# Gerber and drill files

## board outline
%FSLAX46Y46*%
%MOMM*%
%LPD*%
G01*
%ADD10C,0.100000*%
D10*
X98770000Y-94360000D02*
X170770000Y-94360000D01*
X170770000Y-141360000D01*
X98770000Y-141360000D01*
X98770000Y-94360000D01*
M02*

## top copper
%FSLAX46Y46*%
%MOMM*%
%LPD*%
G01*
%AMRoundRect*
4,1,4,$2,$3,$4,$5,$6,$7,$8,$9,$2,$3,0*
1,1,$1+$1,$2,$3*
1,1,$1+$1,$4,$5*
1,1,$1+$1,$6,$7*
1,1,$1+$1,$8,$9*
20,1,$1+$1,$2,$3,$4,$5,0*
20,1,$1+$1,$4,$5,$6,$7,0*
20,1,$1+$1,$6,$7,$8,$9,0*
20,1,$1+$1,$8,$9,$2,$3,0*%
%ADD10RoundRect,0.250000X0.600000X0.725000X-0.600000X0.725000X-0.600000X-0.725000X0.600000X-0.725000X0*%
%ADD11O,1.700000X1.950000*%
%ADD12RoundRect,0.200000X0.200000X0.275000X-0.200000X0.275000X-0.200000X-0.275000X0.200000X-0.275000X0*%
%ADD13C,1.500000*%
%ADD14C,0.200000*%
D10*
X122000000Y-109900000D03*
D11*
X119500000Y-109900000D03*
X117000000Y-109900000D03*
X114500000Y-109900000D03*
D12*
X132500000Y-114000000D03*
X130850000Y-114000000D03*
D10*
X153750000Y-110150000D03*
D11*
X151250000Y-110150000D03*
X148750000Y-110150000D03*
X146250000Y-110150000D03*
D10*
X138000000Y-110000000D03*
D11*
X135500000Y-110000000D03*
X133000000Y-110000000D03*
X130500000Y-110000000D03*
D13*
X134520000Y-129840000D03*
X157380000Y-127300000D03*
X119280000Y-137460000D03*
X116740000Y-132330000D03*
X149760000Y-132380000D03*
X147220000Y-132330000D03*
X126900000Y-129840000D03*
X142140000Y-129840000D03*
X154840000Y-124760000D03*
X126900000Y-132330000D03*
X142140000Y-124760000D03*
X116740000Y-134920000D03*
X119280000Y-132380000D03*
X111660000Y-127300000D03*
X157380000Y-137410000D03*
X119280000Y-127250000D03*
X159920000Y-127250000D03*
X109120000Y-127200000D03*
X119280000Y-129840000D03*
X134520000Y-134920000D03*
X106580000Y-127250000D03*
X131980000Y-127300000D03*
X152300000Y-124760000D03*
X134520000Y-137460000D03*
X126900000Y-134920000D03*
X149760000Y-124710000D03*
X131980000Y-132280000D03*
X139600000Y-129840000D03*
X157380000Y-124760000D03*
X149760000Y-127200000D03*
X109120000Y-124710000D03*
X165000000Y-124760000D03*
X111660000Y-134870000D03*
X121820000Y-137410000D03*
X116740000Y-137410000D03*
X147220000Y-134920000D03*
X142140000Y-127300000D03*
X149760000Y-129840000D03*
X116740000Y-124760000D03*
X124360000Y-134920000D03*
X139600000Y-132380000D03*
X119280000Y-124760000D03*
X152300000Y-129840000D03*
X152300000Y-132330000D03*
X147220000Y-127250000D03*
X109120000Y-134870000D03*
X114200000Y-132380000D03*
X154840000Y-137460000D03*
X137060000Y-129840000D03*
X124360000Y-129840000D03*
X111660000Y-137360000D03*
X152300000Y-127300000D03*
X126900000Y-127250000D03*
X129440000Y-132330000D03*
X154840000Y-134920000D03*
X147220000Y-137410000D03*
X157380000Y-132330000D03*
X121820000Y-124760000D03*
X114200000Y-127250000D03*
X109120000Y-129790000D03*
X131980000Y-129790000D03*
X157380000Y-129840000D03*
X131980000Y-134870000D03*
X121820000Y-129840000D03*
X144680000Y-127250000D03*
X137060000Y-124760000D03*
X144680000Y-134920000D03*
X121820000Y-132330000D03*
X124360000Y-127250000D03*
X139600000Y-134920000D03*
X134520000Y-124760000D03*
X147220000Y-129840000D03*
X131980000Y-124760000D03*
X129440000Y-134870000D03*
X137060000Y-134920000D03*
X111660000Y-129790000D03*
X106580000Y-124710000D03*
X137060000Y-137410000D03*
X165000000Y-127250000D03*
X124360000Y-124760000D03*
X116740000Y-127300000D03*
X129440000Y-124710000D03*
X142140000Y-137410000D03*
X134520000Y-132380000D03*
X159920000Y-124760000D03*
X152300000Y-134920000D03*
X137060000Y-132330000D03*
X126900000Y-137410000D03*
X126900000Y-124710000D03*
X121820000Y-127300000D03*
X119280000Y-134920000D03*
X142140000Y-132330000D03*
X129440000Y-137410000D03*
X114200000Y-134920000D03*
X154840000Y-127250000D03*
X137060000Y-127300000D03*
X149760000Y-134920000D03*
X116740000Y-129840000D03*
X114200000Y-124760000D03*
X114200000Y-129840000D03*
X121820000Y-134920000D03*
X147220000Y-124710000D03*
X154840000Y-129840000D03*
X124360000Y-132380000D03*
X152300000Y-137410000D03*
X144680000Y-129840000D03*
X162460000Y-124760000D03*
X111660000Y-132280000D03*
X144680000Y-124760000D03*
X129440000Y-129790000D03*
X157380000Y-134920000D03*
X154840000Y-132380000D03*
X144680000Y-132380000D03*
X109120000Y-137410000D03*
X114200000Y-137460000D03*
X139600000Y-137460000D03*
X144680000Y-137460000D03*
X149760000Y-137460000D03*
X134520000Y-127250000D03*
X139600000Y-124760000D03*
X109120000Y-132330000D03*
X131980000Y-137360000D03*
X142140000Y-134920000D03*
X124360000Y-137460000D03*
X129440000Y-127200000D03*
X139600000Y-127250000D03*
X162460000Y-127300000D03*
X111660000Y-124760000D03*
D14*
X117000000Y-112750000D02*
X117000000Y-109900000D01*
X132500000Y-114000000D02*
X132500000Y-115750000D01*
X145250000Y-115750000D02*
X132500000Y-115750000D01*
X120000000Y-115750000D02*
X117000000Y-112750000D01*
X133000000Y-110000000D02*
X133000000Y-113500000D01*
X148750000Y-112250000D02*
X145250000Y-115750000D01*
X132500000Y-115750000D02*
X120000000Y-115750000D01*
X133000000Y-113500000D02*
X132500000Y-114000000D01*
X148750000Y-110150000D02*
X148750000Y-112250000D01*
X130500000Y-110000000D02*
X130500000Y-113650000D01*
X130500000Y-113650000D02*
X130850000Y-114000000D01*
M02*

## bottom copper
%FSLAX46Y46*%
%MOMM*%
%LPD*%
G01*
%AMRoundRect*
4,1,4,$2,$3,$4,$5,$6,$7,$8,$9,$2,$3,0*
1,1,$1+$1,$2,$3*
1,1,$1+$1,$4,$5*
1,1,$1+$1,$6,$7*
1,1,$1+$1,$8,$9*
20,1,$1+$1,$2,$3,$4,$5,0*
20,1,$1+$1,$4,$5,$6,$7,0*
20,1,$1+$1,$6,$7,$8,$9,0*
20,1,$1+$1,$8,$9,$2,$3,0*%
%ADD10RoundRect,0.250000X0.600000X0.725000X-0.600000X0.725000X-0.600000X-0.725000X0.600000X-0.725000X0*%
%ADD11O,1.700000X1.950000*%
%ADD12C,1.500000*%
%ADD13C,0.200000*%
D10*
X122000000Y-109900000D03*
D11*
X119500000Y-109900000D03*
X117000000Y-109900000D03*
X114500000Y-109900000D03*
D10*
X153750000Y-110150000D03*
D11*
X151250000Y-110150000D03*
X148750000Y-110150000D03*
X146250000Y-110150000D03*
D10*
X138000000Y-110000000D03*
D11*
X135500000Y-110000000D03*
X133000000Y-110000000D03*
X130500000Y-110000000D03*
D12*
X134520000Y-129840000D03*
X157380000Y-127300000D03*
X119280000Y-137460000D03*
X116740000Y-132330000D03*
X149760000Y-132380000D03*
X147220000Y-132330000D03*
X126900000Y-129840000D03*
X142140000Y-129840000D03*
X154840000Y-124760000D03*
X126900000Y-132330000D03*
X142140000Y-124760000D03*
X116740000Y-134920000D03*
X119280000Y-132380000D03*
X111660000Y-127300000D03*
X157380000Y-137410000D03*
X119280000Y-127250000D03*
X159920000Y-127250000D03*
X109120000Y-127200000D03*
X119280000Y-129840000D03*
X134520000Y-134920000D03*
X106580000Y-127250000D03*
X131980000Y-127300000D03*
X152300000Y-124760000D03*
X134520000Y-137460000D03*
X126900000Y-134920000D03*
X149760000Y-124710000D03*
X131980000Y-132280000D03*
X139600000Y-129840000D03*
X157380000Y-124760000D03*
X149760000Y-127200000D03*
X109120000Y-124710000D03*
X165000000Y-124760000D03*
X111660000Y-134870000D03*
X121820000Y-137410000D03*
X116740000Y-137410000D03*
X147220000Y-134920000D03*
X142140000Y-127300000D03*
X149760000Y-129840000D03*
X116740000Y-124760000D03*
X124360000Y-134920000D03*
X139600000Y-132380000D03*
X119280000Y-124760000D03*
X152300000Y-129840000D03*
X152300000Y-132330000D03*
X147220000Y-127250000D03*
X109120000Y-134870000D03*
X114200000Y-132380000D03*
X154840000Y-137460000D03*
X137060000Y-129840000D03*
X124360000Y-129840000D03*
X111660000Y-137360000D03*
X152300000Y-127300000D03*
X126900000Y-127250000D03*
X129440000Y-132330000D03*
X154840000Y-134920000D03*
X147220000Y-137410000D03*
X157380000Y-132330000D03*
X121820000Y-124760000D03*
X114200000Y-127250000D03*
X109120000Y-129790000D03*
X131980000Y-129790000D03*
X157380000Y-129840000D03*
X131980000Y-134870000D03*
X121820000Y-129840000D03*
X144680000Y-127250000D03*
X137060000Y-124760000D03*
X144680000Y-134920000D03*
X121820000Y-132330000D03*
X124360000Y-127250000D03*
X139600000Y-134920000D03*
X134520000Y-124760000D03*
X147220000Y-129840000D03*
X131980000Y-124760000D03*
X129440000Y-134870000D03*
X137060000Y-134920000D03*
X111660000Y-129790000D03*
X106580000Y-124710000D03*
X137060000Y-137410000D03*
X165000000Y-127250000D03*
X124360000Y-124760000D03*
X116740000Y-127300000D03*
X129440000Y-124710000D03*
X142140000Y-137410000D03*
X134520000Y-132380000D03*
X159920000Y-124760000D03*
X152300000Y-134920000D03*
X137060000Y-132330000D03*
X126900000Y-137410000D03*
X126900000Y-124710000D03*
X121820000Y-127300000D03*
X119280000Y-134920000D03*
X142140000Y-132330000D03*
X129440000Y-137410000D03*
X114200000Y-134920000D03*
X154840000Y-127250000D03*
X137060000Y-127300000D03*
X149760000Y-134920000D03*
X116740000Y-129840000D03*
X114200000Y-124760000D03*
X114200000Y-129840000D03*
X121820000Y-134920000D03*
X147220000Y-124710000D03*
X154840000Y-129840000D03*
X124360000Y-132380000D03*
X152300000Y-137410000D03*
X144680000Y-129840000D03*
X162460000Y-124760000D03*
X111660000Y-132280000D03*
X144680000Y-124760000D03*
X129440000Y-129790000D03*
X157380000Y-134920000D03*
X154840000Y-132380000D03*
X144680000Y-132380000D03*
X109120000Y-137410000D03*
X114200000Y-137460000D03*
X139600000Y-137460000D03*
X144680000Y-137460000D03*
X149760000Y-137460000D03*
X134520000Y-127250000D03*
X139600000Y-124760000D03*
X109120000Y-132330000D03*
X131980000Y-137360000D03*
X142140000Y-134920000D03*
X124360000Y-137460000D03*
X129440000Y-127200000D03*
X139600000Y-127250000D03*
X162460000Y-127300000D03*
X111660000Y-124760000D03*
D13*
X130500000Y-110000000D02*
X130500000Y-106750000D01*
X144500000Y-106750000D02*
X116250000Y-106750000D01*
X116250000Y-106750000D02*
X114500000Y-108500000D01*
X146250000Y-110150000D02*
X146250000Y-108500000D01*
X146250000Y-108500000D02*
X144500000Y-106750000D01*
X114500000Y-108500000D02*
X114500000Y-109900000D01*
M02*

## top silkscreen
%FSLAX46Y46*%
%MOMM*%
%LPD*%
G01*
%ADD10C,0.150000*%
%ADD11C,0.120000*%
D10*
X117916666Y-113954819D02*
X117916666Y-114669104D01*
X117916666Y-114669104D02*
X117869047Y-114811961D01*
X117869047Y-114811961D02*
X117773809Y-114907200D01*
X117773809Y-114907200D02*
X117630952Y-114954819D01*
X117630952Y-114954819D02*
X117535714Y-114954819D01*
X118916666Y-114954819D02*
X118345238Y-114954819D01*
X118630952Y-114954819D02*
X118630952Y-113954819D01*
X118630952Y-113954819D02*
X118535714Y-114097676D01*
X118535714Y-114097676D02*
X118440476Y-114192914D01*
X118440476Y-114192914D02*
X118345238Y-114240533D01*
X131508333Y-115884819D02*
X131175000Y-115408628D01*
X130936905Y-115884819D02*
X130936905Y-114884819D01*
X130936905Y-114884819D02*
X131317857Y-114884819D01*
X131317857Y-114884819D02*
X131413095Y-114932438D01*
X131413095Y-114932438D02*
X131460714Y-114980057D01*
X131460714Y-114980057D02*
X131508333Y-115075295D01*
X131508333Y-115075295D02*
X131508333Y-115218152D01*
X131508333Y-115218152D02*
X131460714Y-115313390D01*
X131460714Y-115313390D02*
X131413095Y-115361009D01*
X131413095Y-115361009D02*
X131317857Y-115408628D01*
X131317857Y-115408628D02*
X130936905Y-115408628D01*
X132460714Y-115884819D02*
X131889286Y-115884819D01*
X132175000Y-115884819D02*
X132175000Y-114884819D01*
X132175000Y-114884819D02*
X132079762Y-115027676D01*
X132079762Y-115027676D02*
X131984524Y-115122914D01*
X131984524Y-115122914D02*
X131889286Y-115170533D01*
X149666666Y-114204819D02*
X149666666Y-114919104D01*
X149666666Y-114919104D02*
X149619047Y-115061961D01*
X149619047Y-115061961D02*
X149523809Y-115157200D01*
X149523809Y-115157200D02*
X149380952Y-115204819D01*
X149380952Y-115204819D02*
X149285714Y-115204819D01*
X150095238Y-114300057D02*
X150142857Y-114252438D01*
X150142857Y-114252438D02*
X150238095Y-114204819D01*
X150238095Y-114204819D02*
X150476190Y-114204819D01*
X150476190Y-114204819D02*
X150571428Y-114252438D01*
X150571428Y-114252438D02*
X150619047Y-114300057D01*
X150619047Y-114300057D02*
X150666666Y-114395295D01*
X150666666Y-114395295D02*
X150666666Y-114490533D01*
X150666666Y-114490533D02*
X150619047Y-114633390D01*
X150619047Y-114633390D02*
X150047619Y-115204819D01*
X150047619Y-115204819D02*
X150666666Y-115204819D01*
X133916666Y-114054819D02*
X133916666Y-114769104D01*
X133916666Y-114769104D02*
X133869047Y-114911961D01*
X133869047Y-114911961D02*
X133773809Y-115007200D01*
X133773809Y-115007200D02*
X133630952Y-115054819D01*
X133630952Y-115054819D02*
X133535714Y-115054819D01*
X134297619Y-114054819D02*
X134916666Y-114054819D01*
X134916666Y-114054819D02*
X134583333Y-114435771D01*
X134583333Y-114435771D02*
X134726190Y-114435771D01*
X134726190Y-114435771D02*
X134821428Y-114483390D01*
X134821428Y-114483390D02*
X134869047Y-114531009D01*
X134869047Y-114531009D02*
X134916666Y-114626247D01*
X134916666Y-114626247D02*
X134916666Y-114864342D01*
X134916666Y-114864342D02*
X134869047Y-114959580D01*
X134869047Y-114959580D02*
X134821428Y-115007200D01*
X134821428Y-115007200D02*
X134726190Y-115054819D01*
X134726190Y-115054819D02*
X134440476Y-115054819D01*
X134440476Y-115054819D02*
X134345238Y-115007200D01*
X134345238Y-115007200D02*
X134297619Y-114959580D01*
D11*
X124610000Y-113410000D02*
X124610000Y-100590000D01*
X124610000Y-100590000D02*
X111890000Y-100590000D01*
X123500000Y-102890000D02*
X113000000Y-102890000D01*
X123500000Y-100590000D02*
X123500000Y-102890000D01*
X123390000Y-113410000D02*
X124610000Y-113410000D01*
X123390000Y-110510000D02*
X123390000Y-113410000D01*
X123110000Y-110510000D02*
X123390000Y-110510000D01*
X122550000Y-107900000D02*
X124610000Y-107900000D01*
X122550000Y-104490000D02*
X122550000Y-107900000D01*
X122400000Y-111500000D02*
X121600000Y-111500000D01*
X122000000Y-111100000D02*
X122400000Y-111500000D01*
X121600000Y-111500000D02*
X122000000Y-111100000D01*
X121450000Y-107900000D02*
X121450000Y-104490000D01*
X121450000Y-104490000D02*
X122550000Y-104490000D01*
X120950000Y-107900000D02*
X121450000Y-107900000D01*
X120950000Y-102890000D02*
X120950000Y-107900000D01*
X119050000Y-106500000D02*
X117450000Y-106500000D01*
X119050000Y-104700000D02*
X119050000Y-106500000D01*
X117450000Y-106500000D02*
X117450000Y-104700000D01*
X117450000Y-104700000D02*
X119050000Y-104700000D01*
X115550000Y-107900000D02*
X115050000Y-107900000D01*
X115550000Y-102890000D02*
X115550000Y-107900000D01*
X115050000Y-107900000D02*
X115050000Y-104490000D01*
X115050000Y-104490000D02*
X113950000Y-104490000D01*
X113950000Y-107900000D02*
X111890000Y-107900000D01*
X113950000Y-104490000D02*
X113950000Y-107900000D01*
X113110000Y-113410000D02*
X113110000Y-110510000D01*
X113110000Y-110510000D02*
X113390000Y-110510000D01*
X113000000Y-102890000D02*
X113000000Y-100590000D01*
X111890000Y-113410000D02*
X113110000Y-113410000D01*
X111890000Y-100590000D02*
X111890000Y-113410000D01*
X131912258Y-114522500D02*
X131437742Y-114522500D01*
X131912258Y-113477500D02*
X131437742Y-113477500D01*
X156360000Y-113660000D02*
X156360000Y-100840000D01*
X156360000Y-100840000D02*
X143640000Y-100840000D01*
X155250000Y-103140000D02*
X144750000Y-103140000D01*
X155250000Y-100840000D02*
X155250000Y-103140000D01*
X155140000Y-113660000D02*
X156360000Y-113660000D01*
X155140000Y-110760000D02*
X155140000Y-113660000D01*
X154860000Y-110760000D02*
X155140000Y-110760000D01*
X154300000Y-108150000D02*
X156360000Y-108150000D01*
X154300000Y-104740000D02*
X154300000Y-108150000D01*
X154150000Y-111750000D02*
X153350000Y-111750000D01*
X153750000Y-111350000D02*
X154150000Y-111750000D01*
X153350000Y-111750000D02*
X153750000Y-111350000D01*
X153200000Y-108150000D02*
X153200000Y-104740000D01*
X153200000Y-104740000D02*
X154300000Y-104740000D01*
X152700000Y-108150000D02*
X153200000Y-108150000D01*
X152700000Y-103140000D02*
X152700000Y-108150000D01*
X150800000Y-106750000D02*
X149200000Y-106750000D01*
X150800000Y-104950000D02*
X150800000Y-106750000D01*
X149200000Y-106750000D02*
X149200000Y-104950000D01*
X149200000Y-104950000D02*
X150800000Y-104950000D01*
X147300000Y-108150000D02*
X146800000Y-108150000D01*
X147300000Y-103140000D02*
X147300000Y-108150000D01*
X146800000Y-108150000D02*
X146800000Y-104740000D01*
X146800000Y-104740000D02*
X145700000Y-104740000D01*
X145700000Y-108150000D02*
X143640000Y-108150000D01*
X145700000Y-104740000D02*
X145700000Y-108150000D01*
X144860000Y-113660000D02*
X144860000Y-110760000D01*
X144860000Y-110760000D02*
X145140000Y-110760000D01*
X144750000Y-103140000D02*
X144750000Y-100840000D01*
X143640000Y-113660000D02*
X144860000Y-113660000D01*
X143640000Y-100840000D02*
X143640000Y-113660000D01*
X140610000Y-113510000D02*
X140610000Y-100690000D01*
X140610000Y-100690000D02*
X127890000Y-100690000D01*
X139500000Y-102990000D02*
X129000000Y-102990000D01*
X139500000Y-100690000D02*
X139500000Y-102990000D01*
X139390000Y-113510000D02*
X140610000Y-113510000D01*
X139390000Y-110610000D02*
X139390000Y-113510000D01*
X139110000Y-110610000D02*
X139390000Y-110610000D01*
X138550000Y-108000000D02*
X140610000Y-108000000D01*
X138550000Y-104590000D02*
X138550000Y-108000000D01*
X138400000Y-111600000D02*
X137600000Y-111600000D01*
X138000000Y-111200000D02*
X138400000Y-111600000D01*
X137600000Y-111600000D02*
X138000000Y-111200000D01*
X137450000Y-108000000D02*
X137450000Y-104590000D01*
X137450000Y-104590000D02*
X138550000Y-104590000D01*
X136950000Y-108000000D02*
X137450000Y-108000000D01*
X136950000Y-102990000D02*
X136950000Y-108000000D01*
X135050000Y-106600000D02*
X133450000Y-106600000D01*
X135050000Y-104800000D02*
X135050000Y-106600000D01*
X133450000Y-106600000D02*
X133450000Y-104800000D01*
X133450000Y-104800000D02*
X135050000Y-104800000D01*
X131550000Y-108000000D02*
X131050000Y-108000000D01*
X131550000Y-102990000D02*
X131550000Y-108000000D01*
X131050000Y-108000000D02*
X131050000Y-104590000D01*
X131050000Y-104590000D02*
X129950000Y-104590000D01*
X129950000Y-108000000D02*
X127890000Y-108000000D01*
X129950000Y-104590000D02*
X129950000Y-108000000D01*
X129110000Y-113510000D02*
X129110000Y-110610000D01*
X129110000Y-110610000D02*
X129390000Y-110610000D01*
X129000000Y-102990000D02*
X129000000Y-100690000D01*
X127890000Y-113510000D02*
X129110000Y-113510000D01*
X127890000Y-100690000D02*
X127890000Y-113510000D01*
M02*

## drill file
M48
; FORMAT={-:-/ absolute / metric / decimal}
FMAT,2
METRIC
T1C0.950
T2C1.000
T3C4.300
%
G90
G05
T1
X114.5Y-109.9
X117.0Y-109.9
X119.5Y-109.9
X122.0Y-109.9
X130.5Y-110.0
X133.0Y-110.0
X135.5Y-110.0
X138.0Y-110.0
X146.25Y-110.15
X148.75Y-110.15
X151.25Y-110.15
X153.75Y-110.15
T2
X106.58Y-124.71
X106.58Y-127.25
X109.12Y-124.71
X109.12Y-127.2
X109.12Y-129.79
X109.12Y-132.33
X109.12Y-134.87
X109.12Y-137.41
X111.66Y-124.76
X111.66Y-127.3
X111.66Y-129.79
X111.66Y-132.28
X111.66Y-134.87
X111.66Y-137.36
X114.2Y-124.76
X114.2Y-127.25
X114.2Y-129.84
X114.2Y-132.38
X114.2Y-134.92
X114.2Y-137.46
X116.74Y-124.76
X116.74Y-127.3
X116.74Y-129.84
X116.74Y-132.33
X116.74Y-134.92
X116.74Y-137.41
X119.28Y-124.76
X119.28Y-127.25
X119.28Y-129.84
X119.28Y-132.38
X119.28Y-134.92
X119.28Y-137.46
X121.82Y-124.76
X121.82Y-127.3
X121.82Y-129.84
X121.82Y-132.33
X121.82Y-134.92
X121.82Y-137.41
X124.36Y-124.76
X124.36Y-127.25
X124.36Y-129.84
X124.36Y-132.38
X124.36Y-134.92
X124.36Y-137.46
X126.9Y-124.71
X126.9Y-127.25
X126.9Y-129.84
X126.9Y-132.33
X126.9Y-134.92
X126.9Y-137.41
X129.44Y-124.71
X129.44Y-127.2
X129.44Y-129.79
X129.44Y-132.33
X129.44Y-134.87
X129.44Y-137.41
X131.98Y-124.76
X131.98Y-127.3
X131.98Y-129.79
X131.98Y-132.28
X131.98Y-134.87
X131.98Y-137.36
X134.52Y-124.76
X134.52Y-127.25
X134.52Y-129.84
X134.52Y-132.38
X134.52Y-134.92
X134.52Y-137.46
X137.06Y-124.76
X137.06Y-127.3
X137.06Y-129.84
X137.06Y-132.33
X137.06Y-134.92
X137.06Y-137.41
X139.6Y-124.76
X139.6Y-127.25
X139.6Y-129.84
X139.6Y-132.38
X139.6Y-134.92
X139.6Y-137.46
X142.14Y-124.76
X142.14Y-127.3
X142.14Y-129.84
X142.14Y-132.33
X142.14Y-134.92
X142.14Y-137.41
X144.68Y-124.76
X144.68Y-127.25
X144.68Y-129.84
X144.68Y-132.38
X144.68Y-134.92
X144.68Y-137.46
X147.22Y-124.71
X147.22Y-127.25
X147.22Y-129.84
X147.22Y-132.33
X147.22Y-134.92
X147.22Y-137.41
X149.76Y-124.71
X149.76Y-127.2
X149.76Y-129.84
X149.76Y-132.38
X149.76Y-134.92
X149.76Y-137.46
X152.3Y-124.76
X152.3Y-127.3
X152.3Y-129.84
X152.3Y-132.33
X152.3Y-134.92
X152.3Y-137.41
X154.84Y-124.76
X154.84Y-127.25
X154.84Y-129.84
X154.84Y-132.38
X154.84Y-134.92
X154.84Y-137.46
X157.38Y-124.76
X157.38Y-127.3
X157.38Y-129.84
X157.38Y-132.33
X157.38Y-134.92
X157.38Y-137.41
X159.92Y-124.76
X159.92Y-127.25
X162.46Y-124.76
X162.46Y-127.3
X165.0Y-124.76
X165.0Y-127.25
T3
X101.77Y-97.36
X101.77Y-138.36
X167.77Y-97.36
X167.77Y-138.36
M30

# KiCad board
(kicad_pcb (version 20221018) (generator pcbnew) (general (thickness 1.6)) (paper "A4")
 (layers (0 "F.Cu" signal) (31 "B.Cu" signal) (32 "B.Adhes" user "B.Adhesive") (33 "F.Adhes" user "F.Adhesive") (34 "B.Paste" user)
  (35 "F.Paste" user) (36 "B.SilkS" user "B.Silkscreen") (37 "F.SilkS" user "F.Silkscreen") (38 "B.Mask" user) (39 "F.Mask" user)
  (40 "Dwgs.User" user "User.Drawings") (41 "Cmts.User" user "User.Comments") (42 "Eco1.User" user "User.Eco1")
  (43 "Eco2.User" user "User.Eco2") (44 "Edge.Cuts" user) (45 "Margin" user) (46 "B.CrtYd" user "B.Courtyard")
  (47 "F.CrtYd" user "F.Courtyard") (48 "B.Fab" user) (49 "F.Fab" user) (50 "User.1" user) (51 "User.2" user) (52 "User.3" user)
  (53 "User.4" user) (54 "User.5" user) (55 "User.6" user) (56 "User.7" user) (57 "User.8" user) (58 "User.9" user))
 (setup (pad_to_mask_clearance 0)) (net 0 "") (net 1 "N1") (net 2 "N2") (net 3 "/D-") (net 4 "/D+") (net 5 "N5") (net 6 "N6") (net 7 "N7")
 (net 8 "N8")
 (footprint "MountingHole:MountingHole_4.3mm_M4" (layer "F.Cu") (at 101.77 138.36)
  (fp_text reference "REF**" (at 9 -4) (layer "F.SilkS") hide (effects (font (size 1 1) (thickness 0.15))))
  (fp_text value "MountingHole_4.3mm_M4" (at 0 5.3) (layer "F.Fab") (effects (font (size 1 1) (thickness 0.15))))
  (pad "" np_thru_hole circle (at 0 0) (size 4.3 4.3) (drill 4.3) (layers "F&B.Cu" "*.Mask")))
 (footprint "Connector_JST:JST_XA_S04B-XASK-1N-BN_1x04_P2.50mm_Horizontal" (layer "F.Cu") (at 122 109.9 180)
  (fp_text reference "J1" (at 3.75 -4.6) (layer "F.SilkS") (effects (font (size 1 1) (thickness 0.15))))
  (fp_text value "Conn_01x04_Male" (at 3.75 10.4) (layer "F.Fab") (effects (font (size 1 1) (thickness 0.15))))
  (fp_line (start -2.61 -3.51) (end -2.61 9.31) (stroke (width 0.12) (type solid)) (layer "F.SilkS"))
  (fp_line (start -2.61 9.31) (end 10.11 9.31) (stroke (width 0.12) (type solid)) (layer "F.SilkS"))
  (fp_line (start -1.5 7.01) (end 9 7.01) (stroke (width 0.12) (type solid)) (layer "F.SilkS"))
  (fp_line (start -1.5 9.31) (end -1.5 7.01) (stroke (width 0.12) (type solid)) (layer "F.SilkS"))
  (fp_line (start -1.39 -3.51) (end -2.61 -3.51) (stroke (width 0.12) (type solid)) (layer "F.SilkS"))
  (fp_line (start -1.39 -0.61) (end -1.39 -3.51) (stroke (width 0.12) (type solid)) (layer "F.SilkS"))
  (fp_line (start -1.11 -0.61) (end -1.39 -0.61) (stroke (width 0.12) (type solid)) (layer "F.SilkS"))
  (fp_line (start -0.55 2) (end -2.61 2) (stroke (width 0.12) (type solid)) (layer "F.SilkS"))
  (fp_line (start -0.55 5.41) (end -0.55 2) (stroke (width 0.12) (type solid)) (layer "F.SilkS"))
  (fp_line (start -0.4 -1.6) (end 0.4 -1.6) (stroke (width 0.12) (type solid)) (layer "F.SilkS"))
  (fp_line (start 0 -1.2) (end -0.4 -1.6) (stroke (width 0.12) (type solid)) (layer "F.SilkS"))
  (fp_line (start 0.4 -1.6) (end 0 -1.2) (stroke (width 0.12) (type solid)) (layer "F.SilkS"))
  (fp_line (start 0.55 2) (end 0.55 5.41) (stroke (width 0.12) (type solid)) (layer "F.SilkS"))
  (fp_line (start 0.55 5.41) (end -0.55 5.41) (stroke (width 0.12) (type solid)) (layer "F.SilkS"))
  (fp_line (start 1.05 2) (end 0.55 2) (stroke (width 0.12) (type solid)) (layer "F.SilkS"))
  (fp_line (start 1.05 7.01) (end 1.05 2) (stroke (width 0.12) (type solid)) (layer "F.SilkS"))
  (fp_line (start 2.95 3.4) (end 4.55 3.4) (stroke (width 0.12) (type solid)) (layer "F.SilkS"))
  (fp_line (start 2.95 5.2) (end 2.95 3.4) (stroke (width 0.12) (type solid)) (layer "F.SilkS"))
  (fp_line (start 4.55 3.4) (end 4.55 5.2) (stroke (width 0.12) (type solid)) (layer "F.SilkS"))
  (fp_line (start 4.55 5.2) (end 2.95 5.2) (stroke (width 0.12) (type solid)) (layer "F.SilkS"))
  (fp_line (start 6.45 2) (end 6.95 2) (stroke (width 0.12) (type solid)) (layer "F.SilkS"))
  (fp_line (start 6.45 7.01) (end 6.45 2) (stroke (width 0.12) (type solid)) (layer "F.SilkS"))
  (fp_line (start 6.95 2) (end 6.95 5.41) (stroke (width 0.12) (type solid)) (layer "F.SilkS"))
  (fp_line (start 6.95 5.41) (end 8.05 5.41) (stroke (width 0.12) (type solid)) (layer "F.SilkS"))
  (fp_line (start 8.05 2) (end 10.11 2) (stroke (width 0.12) (type solid)) (layer "F.SilkS"))
  (fp_line (start 8.05 5.41) (end 8.05 2) (stroke (width 0.12) (type solid)) (layer "F.SilkS"))
  (fp_line (start 8.89 -3.51) (end 8.89 -0.61) (stroke (width 0.12) (type solid)) (layer "F.SilkS"))
  (fp_line (start 8.89 -0.61) (end 8.61 -0.61) (stroke (width 0.12) (type solid)) (layer "F.SilkS"))
  (fp_line (start 9 7.01) (end 9 9.31) (stroke (width 0.12) (type solid)) (layer "F.SilkS"))
  (fp_line (start 10.11 -3.51) (end 8.89 -3.51) (stroke (width 0.12) (type solid)) (layer "F.SilkS"))
  (fp_line (start 10.11 9.31) (end 10.11 -3.51) (stroke (width 0.12) (type solid)) (layer "F.SilkS"))
  (pad "1" thru_hole roundrect (at 0 0 180) (size 1.7 1.95) (drill 0.95) (layers "*.Cu" "*.Mask") (roundrect_rratio 0.147059) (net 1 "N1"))
  (pad "2" thru_hole oval (at 2.5 0 180) (size 1.7 1.95) (drill 0.95) (layers "*.Cu" "*.Mask") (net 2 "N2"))
  (pad "3" thru_hole oval (at 5 0 180) (size 1.7 1.95) (drill 0.95) (layers "*.Cu" "*.Mask") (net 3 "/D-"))
  (pad "4" thru_hole oval (at 7.5 0 180) (size 1.7 1.95) (drill 0.95) (layers "*.Cu" "*.Mask") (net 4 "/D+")))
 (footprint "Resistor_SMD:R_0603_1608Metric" (layer "F.Cu") (at 131.675 114 180)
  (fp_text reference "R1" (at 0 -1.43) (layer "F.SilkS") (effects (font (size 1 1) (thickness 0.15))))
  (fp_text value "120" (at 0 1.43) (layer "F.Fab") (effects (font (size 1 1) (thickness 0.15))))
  (fp_line (start -0.237258 -0.5225) (end 0.237258 -0.5225) (stroke (width 0.12) (type solid)) (layer "F.SilkS"))
  (fp_line (start -0.237258 0.5225) (end 0.237258 0.5225) (stroke (width 0.12) (type solid)) (layer "F.SilkS"))
  (pad "1" smd roundrect (at -0.825 0 180) (size 0.8 0.95) (layers "F.Cu" "F.Paste" "F.Mask") (roundrect_rratio 0.25) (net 3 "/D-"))
  (pad "2" smd roundrect (at 0.825 0 180) (size 0.8 0.95) (layers "F.Cu" "F.Paste" "F.Mask") (roundrect_rratio 0.25) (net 4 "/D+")))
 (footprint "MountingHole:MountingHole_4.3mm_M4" (layer "F.Cu") (at 101.77 97.36)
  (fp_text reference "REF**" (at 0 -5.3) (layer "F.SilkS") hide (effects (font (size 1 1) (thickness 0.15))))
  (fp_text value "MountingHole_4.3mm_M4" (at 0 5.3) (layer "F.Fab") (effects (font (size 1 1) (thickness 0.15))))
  (pad "" np_thru_hole circle (at 0 0) (size 4.3 4.3) (drill 4.3) (layers "F&B.Cu" "*.Mask")))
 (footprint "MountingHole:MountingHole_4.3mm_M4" (layer "F.Cu") (at 167.77 138.36)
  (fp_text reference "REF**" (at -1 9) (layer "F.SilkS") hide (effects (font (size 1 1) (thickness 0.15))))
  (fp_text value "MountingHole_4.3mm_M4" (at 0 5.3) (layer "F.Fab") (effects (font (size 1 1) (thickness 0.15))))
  (pad "" np_thru_hole circle (at 0 0) (size 4.3 4.3) (drill 4.3) (layers "F&B.Cu" "*.Mask")))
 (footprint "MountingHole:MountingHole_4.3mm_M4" (layer "F.Cu") (at 167.77 97.36)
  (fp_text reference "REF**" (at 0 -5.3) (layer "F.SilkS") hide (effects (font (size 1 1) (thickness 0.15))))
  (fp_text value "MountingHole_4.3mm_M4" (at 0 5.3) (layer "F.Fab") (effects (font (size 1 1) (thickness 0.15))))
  (pad "" np_thru_hole circle (at 0 0) (size 4.3 4.3) (drill 4.3) (layers "F&B.Cu" "*.Mask")))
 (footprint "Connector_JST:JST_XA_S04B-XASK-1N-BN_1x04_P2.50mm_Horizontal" (layer "F.Cu") (at 153.75 110.15 180)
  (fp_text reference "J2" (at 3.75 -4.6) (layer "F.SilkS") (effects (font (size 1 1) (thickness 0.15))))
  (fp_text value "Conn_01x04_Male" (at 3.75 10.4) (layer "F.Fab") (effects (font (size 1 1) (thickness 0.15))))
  (fp_line (start -2.61 -3.51) (end -2.61 9.31) (stroke (width 0.12) (type solid)) (layer "F.SilkS"))
  (fp_line (start -2.61 9.31) (end 10.11 9.31) (stroke (width 0.12) (type solid)) (layer "F.SilkS"))
  (fp_line (start -1.5 7.01) (end 9 7.01) (stroke (width 0.12) (type solid)) (layer "F.SilkS"))
  (fp_line (start -1.5 9.31) (end -1.5 7.01) (stroke (width 0.12) (type solid)) (layer "F.SilkS"))
  (fp_line (start -1.39 -3.51) (end -2.61 -3.51) (stroke (width 0.12) (type solid)) (layer "F.SilkS"))
  (fp_line (start -1.39 -0.61) (end -1.39 -3.51) (stroke (width 0.12) (type solid)) (layer "F.SilkS"))
  (fp_line (start -1.11 -0.61) (end -1.39 -0.61) (stroke (width 0.12) (type solid)) (layer "F.SilkS"))
  (fp_line (start -0.55 2) (end -2.61 2) (stroke (width 0.12) (type solid)) (layer "F.SilkS"))
  (fp_line (start -0.55 5.41) (end -0.55 2) (stroke (width 0.12) (type solid)) (layer "F.SilkS"))
  (fp_line (start -0.4 -1.6) (end 0.4 -1.6) (stroke (width 0.12) (type solid)) (layer "F.SilkS"))
  (fp_line (start 0 -1.2) (end -0.4 -1.6) (stroke (width 0.12) (type solid)) (layer "F.SilkS"))
  (fp_line (start 0.4 -1.6) (end 0 -1.2) (stroke (width 0.12) (type solid)) (layer "F.SilkS"))
  (fp_line (start 0.55 2) (end 0.55 5.41) (stroke (width 0.12) (type solid)) (layer "F.SilkS"))
  (fp_line (start 0.55 5.41) (end -0.55 5.41) (stroke (width 0.12) (type solid)) (layer "F.SilkS"))
  (fp_line (start 1.05 2) (end 0.55 2) (stroke (width 0.12) (type solid)) (layer "F.SilkS"))
  (fp_line (start 1.05 7.01) (end 1.05 2) (stroke (width 0.12) (type solid)) (layer "F.SilkS"))
  (fp_line (start 2.95 3.4) (end 4.55 3.4) (stroke (width 0.12) (type solid)) (layer "F.SilkS"))
  (fp_line (start 2.95 5.2) (end 2.95 3.4) (stroke (width 0.12) (type solid)) (layer "F.SilkS"))
  (fp_line (start 4.55 3.4) (end 4.55 5.2) (stroke (width 0.12) (type solid)) (layer "F.SilkS"))
  (fp_line (start 4.55 5.2) (end 2.95 5.2) (stroke (width 0.12) (type solid)) (layer "F.SilkS"))
  (fp_line (start 6.45 2) (end 6.95 2) (stroke (width 0.12) (type solid)) (layer "F.SilkS"))
  (fp_line (start 6.45 7.01) (end 6.45 2) (stroke (width 0.12) (type solid)) (layer "F.SilkS"))
  (fp_line (start 6.95 2) (end 6.95 5.41) (stroke (width 0.12) (type solid)) (layer "F.SilkS"))
  (fp_line (start 6.95 5.41) (end 8.05 5.41) (stroke (width 0.12) (type solid)) (layer "F.SilkS"))
  (fp_line (start 8.05 2) (end 10.11 2) (stroke (width 0.12) (type solid)) (layer "F.SilkS"))
  (fp_line (start 8.05 5.41) (end 8.05 2) (stroke (width 0.12) (type solid)) (layer "F.SilkS"))
  (fp_line (start 8.89 -3.51) (end 8.89 -0.61) (stroke (width 0.12) (type solid)) (layer "F.SilkS"))
  (fp_line (start 8.89 -0.61) (end 8.61 -0.61) (stroke (width 0.12) (type solid)) (layer "F.SilkS"))
  (fp_line (start 9 7.01) (end 9 9.31) (stroke (width 0.12) (type solid)) (layer "F.SilkS"))
  (fp_line (start 10.11 -3.51) (end 8.89 -3.51) (stroke (width 0.12) (type solid)) (layer "F.SilkS"))
  (fp_line (start 10.11 9.31) (end 10.11 -3.51) (stroke (width 0.12) (type solid)) (layer "F.SilkS"))
  (pad "1" thru_hole roundrect (at 0 0 180) (size 1.7 1.95) (drill 0.95) (layers "*.Cu" "*.Mask") (roundrect_rratio 0.147059) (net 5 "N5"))
  (pad "2" thru_hole oval (at 2.5 0 180) (size 1.7 1.95) (drill 0.95) (layers "*.Cu" "*.Mask") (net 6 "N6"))
  (pad "3" thru_hole oval (at 5 0 180) (size 1.7 1.95) (drill 0.95) (layers "*.Cu" "*.Mask") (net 3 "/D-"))
  (pad "4" thru_hole oval (at 7.5 0 180) (size 1.7 1.95) (drill 0.95) (layers "*.Cu" "*.Mask") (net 4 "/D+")))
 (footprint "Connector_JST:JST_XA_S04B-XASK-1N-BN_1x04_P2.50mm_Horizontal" (layer "F.Cu") (at 138 110 180)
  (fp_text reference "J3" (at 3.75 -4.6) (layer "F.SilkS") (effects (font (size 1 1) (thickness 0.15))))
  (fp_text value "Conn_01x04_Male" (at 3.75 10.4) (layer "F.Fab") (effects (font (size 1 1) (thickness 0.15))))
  (fp_line (start -2.61 -3.51) (end -2.61 9.31) (stroke (width 0.12) (type solid)) (layer "F.SilkS"))
  (fp_line (start -2.61 9.31) (end 10.11 9.31) (stroke (width 0.12) (type solid)) (layer "F.SilkS"))
  (fp_line (start -1.5 7.01) (end 9 7.01) (stroke (width 0.12) (type solid)) (layer "F.SilkS"))
  (fp_line (start -1.5 9.31) (end -1.5 7.01) (stroke (width 0.12) (type solid)) (layer "F.SilkS"))
  (fp_line (start -1.39 -3.51) (end -2.61 -3.51) (stroke (width 0.12) (type solid)) (layer "F.SilkS"))
  (fp_line (start -1.39 -0.61) (end -1.39 -3.51) (stroke (width 0.12) (type solid)) (layer "F.SilkS"))
  (fp_line (start -1.11 -0.61) (end -1.39 -0.61) (stroke (width 0.12) (type solid)) (layer "F.SilkS"))
  (fp_line (start -0.55 2) (end -2.61 2) (stroke (width 0.12) (type solid)) (layer "F.SilkS"))
  (fp_line (start -0.55 5.41) (end -0.55 2) (stroke (width 0.12) (type solid)) (layer "F.SilkS"))
  (fp_line (start -0.4 -1.6) (end 0.4 -1.6) (stroke (width 0.12) (type solid)) (layer "F.SilkS"))
  (fp_line (start 0 -1.2) (end -0.4 -1.6) (stroke (width 0.12) (type solid)) (layer "F.SilkS"))
  (fp_line (start 0.4 -1.6) (end 0 -1.2) (stroke (width 0.12) (type solid)) (layer "F.SilkS"))
  (fp_line (start 0.55 2) (end 0.55 5.41) (stroke (width 0.12) (type solid)) (layer "F.SilkS"))
  (fp_line (start 0.55 5.41) (end -0.55 5.41) (stroke (width 0.12) (type solid)) (layer "F.SilkS"))
  (fp_line (start 1.05 2) (end 0.55 2) (stroke (width 0.12) (type solid)) (layer "F.SilkS"))
  (fp_line (start 1.05 7.01) (end 1.05 2) (stroke (width 0.12) (type solid)) (layer "F.SilkS"))
  (fp_line (start 2.95 3.4) (end 4.55 3.4) (stroke (width 0.12) (type solid)) (layer "F.SilkS"))
  (fp_line (start 2.95 5.2) (end 2.95 3.4) (stroke (width 0.12) (type solid)) (layer "F.SilkS"))
  (fp_line (start 4.55 3.4) (end 4.55 5.2) (stroke (width 0.12) (type solid)) (layer "F.SilkS"))
  (fp_line (start 4.55 5.2) (end 2.95 5.2) (stroke (width 0.12) (type solid)) (layer "F.SilkS"))
  (fp_line (start 6.45 2) (end 6.95 2) (stroke (width 0.12) (type solid)) (layer "F.SilkS"))
  (fp_line (start 6.45 7.01) (end 6.45 2) (stroke (width 0.12) (type solid)) (layer "F.SilkS"))
  (fp_line (start 6.95 2) (end 6.95 5.41) (stroke (width 0.12) (type solid)) (layer "F.SilkS"))
  (fp_line (start 6.95 5.41) (end 8.05 5.41) (stroke (width 0.12) (type solid)) (layer "F.SilkS"))
  (fp_line (start 8.05 2) (end 10.11 2) (stroke (width 0.12) (type solid)) (layer "F.SilkS"))
  (fp_line (start 8.05 5.41) (end 8.05 2) (stroke (width 0.12) (type solid)) (layer "F.SilkS"))
  (fp_line (start 8.89 -3.51) (end 8.89 -0.61) (stroke (width 0.12) (type solid)) (layer "F.SilkS"))
  (fp_line (start 8.89 -0.61) (end 8.61 -0.61) (stroke (width 0.12) (type solid)) (layer "F.SilkS"))
  (fp_line (start 9 7.01) (end 9 9.31) (stroke (width 0.12) (type solid)) (layer "F.SilkS"))
  (fp_line (start 10.11 -3.51) (end 8.89 -3.51) (stroke (width 0.12) (type solid)) (layer "F.SilkS"))
  (fp_line (start 10.11 9.31) (end 10.11 -3.51) (stroke (width 0.12) (type solid)) (layer "F.SilkS"))
  (pad "1" thru_hole roundrect (at 0 0 180) (size 1.7 1.95) (drill 0.95) (layers "*.Cu" "*.Mask") (roundrect_rratio 0.147059) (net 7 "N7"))
  (pad "2" thru_hole oval (at 2.5 0 180) (size 1.7 1.95) (drill 0.95) (layers "*.Cu" "*.Mask") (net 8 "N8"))
  (pad "3" thru_hole oval (at 5 0 180) (size 1.7 1.95) (drill 0.95) (layers "*.Cu" "*.Mask") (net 3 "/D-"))
  (pad "4" thru_hole oval (at 7.5 0 180) (size 1.7 1.95) (drill 0.95) (layers "*.Cu" "*.Mask") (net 4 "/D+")))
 (gr_rect (start 98.77 94.36) (end 170.77 141.36) (stroke (width 0.1) (type solid)) (fill none) (layer "Edge.Cuts"))
 (via (at 134.52 129.84) (size 1.5) (drill 1) (layers "F.Cu" "B.Cu") (free) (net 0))
 (via (at 157.38 127.3) (size 1.5) (drill 1) (layers "F.Cu" "B.Cu") (free) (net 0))
 (via (at 119.28 137.46) (size 1.5) (drill 1) (layers "F.Cu" "B.Cu") (free) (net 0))
 (via (at 116.74 132.33) (size 1.5) (drill 1) (layers "F.Cu" "B.Cu") (free) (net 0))
 (via (at 149.76 132.38) (size 1.5) (drill 1) (layers "F.Cu" "B.Cu") (free) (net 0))
 (via (at 147.22 132.33) (size 1.5) (drill 1) (layers "F.Cu" "B.Cu") (free) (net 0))
 (via (at 126.9 129.84) (size 1.5) (drill 1) (layers "F.Cu" "B.Cu") (free) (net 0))
 (via (at 142.14 129.84) (size 1.5) (drill 1) (layers "F.Cu" "B.Cu") (free) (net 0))
 (via (at 154.84 124.76) (size 1.5) (drill 1) (layers "F.Cu" "B.Cu") (free) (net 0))
 (via (at 126.9 132.33) (size 1.5) (drill 1) (layers "F.Cu" "B.Cu") (free) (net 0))
 (via (at 142.14 124.76) (size 1.5) (drill 1) (layers "F.Cu" "B.Cu") (free) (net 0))
 (via (at 116.74 134.92) (size 1.5) (drill 1) (layers "F.Cu" "B.Cu") (free) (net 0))
 (via (at 119.28 132.38) (size 1.5) (drill 1) (layers "F.Cu" "B.Cu") (free) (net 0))
 (via (at 111.66 127.3) (size 1.5) (drill 1) (layers "F.Cu" "B.Cu") (free) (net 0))
 (via (at 157.38 137.41) (size 1.5) (drill 1) (layers "F.Cu" "B.Cu") (free) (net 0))
 (via (at 119.28 127.25) (size 1.5) (drill 1) (layers "F.Cu" "B.Cu") (free) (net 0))
 (via (at 159.92 127.25) (size 1.5) (drill 1) (layers "F.Cu" "B.Cu") (free) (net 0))
 (via (at 109.12 127.2) (size 1.5) (drill 1) (layers "F.Cu" "B.Cu") (free) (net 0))
 (via (at 119.28 129.84) (size 1.5) (drill 1) (layers "F.Cu" "B.Cu") (free) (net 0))
 (via (at 134.52 134.92) (size 1.5) (drill 1) (layers "F.Cu" "B.Cu") (free) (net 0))
 (via (at 106.58 127.25) (size 1.5) (drill 1) (layers "F.Cu" "B.Cu") (free) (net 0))
 (via (at 131.98 127.3) (size 1.5) (drill 1) (layers "F.Cu" "B.Cu") (free) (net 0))
 (via (at 152.3 124.76) (size 1.5) (drill 1) (layers "F.Cu" "B.Cu") (free) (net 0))
 (via (at 134.52 137.46) (size 1.5) (drill 1) (layers "F.Cu" "B.Cu") (free) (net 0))
 (via (at 126.9 134.92) (size 1.5) (drill 1) (layers "F.Cu" "B.Cu") (free) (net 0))
 (via (at 149.76 124.71) (size 1.5) (drill 1) (layers "F.Cu" "B.Cu") (free) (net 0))
 (via (at 131.98 132.28) (size 1.5) (drill 1) (layers "F.Cu" "B.Cu") (free) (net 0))
 (via (at 139.6 129.84) (size 1.5) (drill 1) (layers "F.Cu" "B.Cu") (free) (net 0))
 (via (at 157.38 124.76) (size 1.5) (drill 1) (layers "F.Cu" "B.Cu") (free) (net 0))
 (via (at 149.76 127.2) (size 1.5) (drill 1) (layers "F.Cu" "B.Cu") (free) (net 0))
 (via (at 109.12 124.71) (size 1.5) (drill 1) (layers "F.Cu" "B.Cu") (free) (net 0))
 (via (at 165 124.76) (size 1.5) (drill 1) (layers "F.Cu" "B.Cu") (free) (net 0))
 (via (at 111.66 134.87) (size 1.5) (drill 1) (layers "F.Cu" "B.Cu") (free) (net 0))
 (via (at 121.82 137.41) (size 1.5) (drill 1) (layers "F.Cu" "B.Cu") (free) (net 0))
 (via (at 116.74 137.41) (size 1.5) (drill 1) (layers "F.Cu" "B.Cu") (free) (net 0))
 (via (at 147.22 134.92) (size 1.5) (drill 1) (layers "F.Cu" "B.Cu") (free) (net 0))
 (via (at 142.14 127.3) (size 1.5) (drill 1) (layers "F.Cu" "B.Cu") (free) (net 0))
 (via (at 149.76 129.84) (size 1.5) (drill 1) (layers "F.Cu" "B.Cu") (free) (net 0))
 (via (at 116.74 124.76) (size 1.5) (drill 1) (layers "F.Cu" "B.Cu") (free) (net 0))
 (via (at 124.36 134.92) (size 1.5) (drill 1) (layers "F.Cu" "B.Cu") (free) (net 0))
 (via (at 139.6 132.38) (size 1.5) (drill 1) (layers "F.Cu" "B.Cu") (free) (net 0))
 (via (at 119.28 124.76) (size 1.5) (drill 1) (layers "F.Cu" "B.Cu") (free) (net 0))
 (via (at 152.3 129.84) (size 1.5) (drill 1) (layers "F.Cu" "B.Cu") (free) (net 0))
 (via (at 152.3 132.33) (size 1.5) (drill 1) (layers "F.Cu" "B.Cu") (free) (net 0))
 (via (at 147.22 127.25) (size 1.5) (drill 1) (layers "F.Cu" "B.Cu") (free) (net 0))
 (via (at 109.12 134.87) (size 1.5) (drill 1) (layers "F.Cu" "B.Cu") (free) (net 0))
 (via (at 114.2 132.38) (size 1.5) (drill 1) (layers "F.Cu" "B.Cu") (free) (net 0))
 (via (at 154.84 137.46) (size 1.5) (drill 1) (layers "F.Cu" "B.Cu") (free) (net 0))
 (via (at 137.06 129.84) (size 1.5) (drill 1) (layers "F.Cu" "B.Cu") (free) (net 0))
 (via (at 124.36 129.84) (size 1.5) (drill 1) (layers "F.Cu" "B.Cu") (free) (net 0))
 (via (at 111.66 137.36) (size 1.5) (drill 1) (layers "F.Cu" "B.Cu") (free) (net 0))
 (via (at 152.3 127.3) (size 1.5) (drill 1) (layers "F.Cu" "B.Cu") (free) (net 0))
 (via (at 126.9 127.25) (size 1.5) (drill 1) (layers "F.Cu" "B.Cu") (free) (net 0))
 (via (at 129.44 132.33) (size 1.5) (drill 1) (layers "F.Cu" "B.Cu") (free) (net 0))
 (via (at 154.84 134.92) (size 1.5) (drill 1) (layers "F.Cu" "B.Cu") (free) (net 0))
 (via (at 147.22 137.41) (size 1.5) (drill 1) (layers "F.Cu" "B.Cu") (free) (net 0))
 (via (at 157.38 132.33) (size 1.5) (drill 1) (layers "F.Cu" "B.Cu") (free) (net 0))
 (via (at 121.82 124.76) (size 1.5) (drill 1) (layers "F.Cu" "B.Cu") (free) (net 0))
 (via (at 114.2 127.25) (size 1.5) (drill 1) (layers "F.Cu" "B.Cu") (free) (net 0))
 (via (at 109.12 129.79) (size 1.5) (drill 1) (layers "F.Cu" "B.Cu") (free) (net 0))
 (via (at 131.98 129.79) (size 1.5) (drill 1) (layers "F.Cu" "B.Cu") (free) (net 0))
 (via (at 157.38 129.84) (size 1.5) (drill 1) (layers "F.Cu" "B.Cu") (free) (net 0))
 (via (at 131.98 134.87) (size 1.5) (drill 1) (layers "F.Cu" "B.Cu") (free) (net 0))
 (via (at 121.82 129.84) (size 1.5) (drill 1) (layers "F.Cu" "B.Cu") (free) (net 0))
 (via (at 144.68 127.25) (size 1.5) (drill 1) (layers "F.Cu" "B.Cu") (free) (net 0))
 (via (at 137.06 124.76) (size 1.5) (drill 1) (layers "F.Cu" "B.Cu") (free) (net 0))
 (via (at 144.68 134.92) (size 1.5) (drill 1) (layers "F.Cu" "B.Cu") (free) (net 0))
 (via (at 121.82 132.33) (size 1.5) (drill 1) (layers "F.Cu" "B.Cu") (free) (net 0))
 (via (at 124.36 127.25) (size 1.5) (drill 1) (layers "F.Cu" "B.Cu") (free) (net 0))
 (via (at 139.6 134.92) (size 1.5) (drill 1) (layers "F.Cu" "B.Cu") (free) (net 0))
 (via (at 134.52 124.76) (size 1.5) (drill 1) (layers "F.Cu" "B.Cu") (free) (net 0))
 (via (at 147.22 129.84) (size 1.5) (drill 1) (layers "F.Cu" "B.Cu") (free) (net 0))
 (via (at 131.98 124.76) (size 1.5) (drill 1) (layers "F.Cu" "B.Cu") (free) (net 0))
 (via (at 129.44 134.87) (size 1.5) (drill 1) (layers "F.Cu" "B.Cu") (free) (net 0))
 (via (at 137.06 134.92) (size 1.5) (drill 1) (layers "F.Cu" "B.Cu") (free) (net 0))
 (via (at 111.66 129.79) (size 1.5) (drill 1) (layers "F.Cu" "B.Cu") (free) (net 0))
 (via (at 106.58 124.71) (size 1.5) (drill 1) (layers "F.Cu" "B.Cu") (free) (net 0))
 (via (at 137.06 137.41) (size 1.5) (drill 1) (layers "F.Cu" "B.Cu") (free) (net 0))
 (via (at 165 127.25) (size 1.5) (drill 1) (layers "F.Cu" "B.Cu") (free) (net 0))
 (via (at 124.36 124.76) (size 1.5) (drill 1) (layers "F.Cu" "B.Cu") (free) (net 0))
 (via (at 116.74 127.3) (size 1.5) (drill 1) (layers "F.Cu" "B.Cu") (free) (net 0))
 (via (at 129.44 124.71) (size 1.5) (drill 1) (layers "F.Cu" "B.Cu") (free) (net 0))
 (via (at 142.14 137.41) (size 1.5) (drill 1) (layers "F.Cu" "B.Cu") (free) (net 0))
 (via (at 134.52 132.38) (size 1.5) (drill 1) (layers "F.Cu" "B.Cu") (free) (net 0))
 (via (at 159.92 124.76) (size 1.5) (drill 1) (layers "F.Cu" "B.Cu") (free) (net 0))
 (via (at 152.3 134.92) (size 1.5) (drill 1) (layers "F.Cu" "B.Cu") (free) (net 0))
 (via (at 137.06 132.33) (size 1.5) (drill 1) (layers "F.Cu" "B.Cu") (free) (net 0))
 (via (at 126.9 137.41) (size 1.5) (drill 1) (layers "F.Cu" "B.Cu") (free) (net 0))
 (via (at 126.9 124.71) (size 1.5) (drill 1) (layers "F.Cu" "B.Cu") (free) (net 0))
 (via (at 121.82 127.3) (size 1.5) (drill 1) (layers "F.Cu" "B.Cu") (free) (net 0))
 (via (at 119.28 134.92) (size 1.5) (drill 1) (layers "F.Cu" "B.Cu") (free) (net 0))
 (via (at 142.14 132.33) (size 1.5) (drill 1) (layers "F.Cu" "B.Cu") (free) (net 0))
 (via (at 129.44 137.41) (size 1.5) (drill 1) (layers "F.Cu" "B.Cu") (free) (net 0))
 (via (at 114.2 134.92) (size 1.5) (drill 1) (layers "F.Cu" "B.Cu") (free) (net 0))
 (via (at 154.84 127.25) (size 1.5) (drill 1) (layers "F.Cu" "B.Cu") (free) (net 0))
 (via (at 137.06 127.3) (size 1.5) (drill 1) (layers "F.Cu" "B.Cu") (free) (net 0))
 (via (at 149.76 134.92) (size 1.5) (drill 1) (layers "F.Cu" "B.Cu") (free) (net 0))
 (via (at 116.74 129.84) (size 1.5) (drill 1) (layers "F.Cu" "B.Cu") (free) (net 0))
 (via (at 114.2 124.76) (size 1.5) (drill 1) (layers "F.Cu" "B.Cu") (free) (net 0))
 (via (at 114.2 129.84) (size 1.5) (drill 1) (layers "F.Cu" "B.Cu") (free) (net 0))
 (via (at 121.82 134.92) (size 1.5) (drill 1) (layers "F.Cu" "B.Cu") (free) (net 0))
 (via (at 147.22 124.71) (size 1.5) (drill 1) (layers "F.Cu" "B.Cu") (free) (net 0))
 (via (at 154.84 129.84) (size 1.5) (drill 1) (layers "F.Cu" "B.Cu") (free) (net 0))
 (via (at 124.36 132.38) (size 1.5) (drill 1) (layers "F.Cu" "B.Cu") (free) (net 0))
 (via (at 152.3 137.41) (size 1.5) (drill 1) (layers "F.Cu" "B.Cu") (free) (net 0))
 (via (at 144.68 129.84) (size 1.5) (drill 1) (layers "F.Cu" "B.Cu") (free) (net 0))
 (via (at 162.46 124.76) (size 1.5) (drill 1) (layers "F.Cu" "B.Cu") (free) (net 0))
 (via (at 111.66 132.28) (size 1.5) (drill 1) (layers "F.Cu" "B.Cu") (free) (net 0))
 (via (at 144.68 124.76) (size 1.5) (drill 1) (layers "F.Cu" "B.Cu") (free) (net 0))
 (via (at 129.44 129.79) (size 1.5) (drill 1) (layers "F.Cu" "B.Cu") (free) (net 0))
 (via (at 157.38 134.92) (size 1.5) (drill 1) (layers "F.Cu" "B.Cu") (free) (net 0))
 (via (at 154.84 132.38) (size 1.5) (drill 1) (layers "F.Cu" "B.Cu") (free) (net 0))
 (via (at 144.68 132.38) (size 1.5) (drill 1) (layers "F.Cu" "B.Cu") (free) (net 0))
 (via (at 109.12 137.41) (size 1.5) (drill 1) (layers "F.Cu" "B.Cu") (free) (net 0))
 (via (at 114.2 137.46) (size 1.5) (drill 1) (layers "F.Cu" "B.Cu") (free) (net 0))
 (via (at 139.6 137.46) (size 1.5) (drill 1) (layers "F.Cu" "B.Cu") (free) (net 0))
 (via (at 144.68 137.46) (size 1.5) (drill 1) (layers "F.Cu" "B.Cu") (free) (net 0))
 (via (at 149.76 137.46) (size 1.5) (drill 1) (layers "F.Cu" "B.Cu") (free) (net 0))
 (via (at 134.52 127.25) (size 1.5) (drill 1) (layers "F.Cu" "B.Cu") (free) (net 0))
 (via (at 139.6 124.76) (size 1.5) (drill 1) (layers "F.Cu" "B.Cu") (free) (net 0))
 (via (at 109.12 132.33) (size 1.5) (drill 1) (layers "F.Cu" "B.Cu") (free) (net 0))
 (via (at 131.98 137.36) (size 1.5) (drill 1) (layers "F.Cu" "B.Cu") (free) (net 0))
 (via (at 142.14 134.92) (size 1.5) (drill 1) (layers "F.Cu" "B.Cu") (free) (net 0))
 (via (at 124.36 137.46) (size 1.5) (drill 1) (layers "F.Cu" "B.Cu") (free) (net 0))
 (via (at 129.44 127.2) (size 1.5) (drill 1) (layers "F.Cu" "B.Cu") (free) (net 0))
 (via (at 139.6 127.25) (size 1.5) (drill 1) (layers "F.Cu" "B.Cu") (free) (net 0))
 (via (at 162.46 127.3) (size 1.5) (drill 1) (layers "F.Cu" "B.Cu") (free) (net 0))
 (via (at 111.66 124.76) (size 1.5) (drill 1) (layers "F.Cu" "B.Cu") (free) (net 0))
 (segment (start 117 112.75) (end 117 109.9) (width 0.2) (layer "F.Cu") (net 3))
 (segment (start 132.5 114) (end 132.5 115.75) (width 0.2) (layer "F.Cu") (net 3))
 (segment (start 145.25 115.75) (end 132.5 115.75) (width 0.2) (layer "F.Cu") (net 3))
 (segment (start 120 115.75) (end 117 112.75) (width 0.2) (layer "F.Cu") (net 3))
 (segment (start 133 110) (end 133 113.5) (width 0.2) (layer "F.Cu") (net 3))
 (segment (start 148.75 112.25) (end 145.25 115.75) (width 0.2) (layer "F.Cu") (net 3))
 (segment (start 132.5 115.75) (end 120 115.75) (width 0.2) (layer "F.Cu") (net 3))
 (segment (start 133 113.5) (end 132.5 114) (width 0.2) (layer "F.Cu") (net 3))
 (segment (start 148.75 110.15) (end 148.75 112.25) (width 0.2) (layer "F.Cu") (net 3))
 (segment (start 130.5 110) (end 130.5 113.65) (width 0.2) (layer "F.Cu") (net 4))
 (segment (start 130.5 113.65) (end 130.85 114) (width 0.2) (layer "F.Cu") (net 4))
 (segment (start 130.5 110) (end 130.5 106.75) (width 0.2) (layer "B.Cu") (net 4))
 (segment (start 144.5 106.75) (end 116.25 106.75) (width 0.2) (layer "B.Cu") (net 4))
 (segment (start 116.25 106.75) (end 114.5 108.5) (width 0.2) (layer "B.Cu") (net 4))
 (segment (start 146.25 110.15) (end 146.25 108.5) (width 0.2) (layer "B.Cu") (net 4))
 (segment (start 146.25 108.5) (end 144.5 106.75) (width 0.2) (layer "B.Cu") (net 4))
 (segment (start 114.5 108.5) (end 114.5 109.9) (width 0.2) (layer "B.Cu") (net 4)))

